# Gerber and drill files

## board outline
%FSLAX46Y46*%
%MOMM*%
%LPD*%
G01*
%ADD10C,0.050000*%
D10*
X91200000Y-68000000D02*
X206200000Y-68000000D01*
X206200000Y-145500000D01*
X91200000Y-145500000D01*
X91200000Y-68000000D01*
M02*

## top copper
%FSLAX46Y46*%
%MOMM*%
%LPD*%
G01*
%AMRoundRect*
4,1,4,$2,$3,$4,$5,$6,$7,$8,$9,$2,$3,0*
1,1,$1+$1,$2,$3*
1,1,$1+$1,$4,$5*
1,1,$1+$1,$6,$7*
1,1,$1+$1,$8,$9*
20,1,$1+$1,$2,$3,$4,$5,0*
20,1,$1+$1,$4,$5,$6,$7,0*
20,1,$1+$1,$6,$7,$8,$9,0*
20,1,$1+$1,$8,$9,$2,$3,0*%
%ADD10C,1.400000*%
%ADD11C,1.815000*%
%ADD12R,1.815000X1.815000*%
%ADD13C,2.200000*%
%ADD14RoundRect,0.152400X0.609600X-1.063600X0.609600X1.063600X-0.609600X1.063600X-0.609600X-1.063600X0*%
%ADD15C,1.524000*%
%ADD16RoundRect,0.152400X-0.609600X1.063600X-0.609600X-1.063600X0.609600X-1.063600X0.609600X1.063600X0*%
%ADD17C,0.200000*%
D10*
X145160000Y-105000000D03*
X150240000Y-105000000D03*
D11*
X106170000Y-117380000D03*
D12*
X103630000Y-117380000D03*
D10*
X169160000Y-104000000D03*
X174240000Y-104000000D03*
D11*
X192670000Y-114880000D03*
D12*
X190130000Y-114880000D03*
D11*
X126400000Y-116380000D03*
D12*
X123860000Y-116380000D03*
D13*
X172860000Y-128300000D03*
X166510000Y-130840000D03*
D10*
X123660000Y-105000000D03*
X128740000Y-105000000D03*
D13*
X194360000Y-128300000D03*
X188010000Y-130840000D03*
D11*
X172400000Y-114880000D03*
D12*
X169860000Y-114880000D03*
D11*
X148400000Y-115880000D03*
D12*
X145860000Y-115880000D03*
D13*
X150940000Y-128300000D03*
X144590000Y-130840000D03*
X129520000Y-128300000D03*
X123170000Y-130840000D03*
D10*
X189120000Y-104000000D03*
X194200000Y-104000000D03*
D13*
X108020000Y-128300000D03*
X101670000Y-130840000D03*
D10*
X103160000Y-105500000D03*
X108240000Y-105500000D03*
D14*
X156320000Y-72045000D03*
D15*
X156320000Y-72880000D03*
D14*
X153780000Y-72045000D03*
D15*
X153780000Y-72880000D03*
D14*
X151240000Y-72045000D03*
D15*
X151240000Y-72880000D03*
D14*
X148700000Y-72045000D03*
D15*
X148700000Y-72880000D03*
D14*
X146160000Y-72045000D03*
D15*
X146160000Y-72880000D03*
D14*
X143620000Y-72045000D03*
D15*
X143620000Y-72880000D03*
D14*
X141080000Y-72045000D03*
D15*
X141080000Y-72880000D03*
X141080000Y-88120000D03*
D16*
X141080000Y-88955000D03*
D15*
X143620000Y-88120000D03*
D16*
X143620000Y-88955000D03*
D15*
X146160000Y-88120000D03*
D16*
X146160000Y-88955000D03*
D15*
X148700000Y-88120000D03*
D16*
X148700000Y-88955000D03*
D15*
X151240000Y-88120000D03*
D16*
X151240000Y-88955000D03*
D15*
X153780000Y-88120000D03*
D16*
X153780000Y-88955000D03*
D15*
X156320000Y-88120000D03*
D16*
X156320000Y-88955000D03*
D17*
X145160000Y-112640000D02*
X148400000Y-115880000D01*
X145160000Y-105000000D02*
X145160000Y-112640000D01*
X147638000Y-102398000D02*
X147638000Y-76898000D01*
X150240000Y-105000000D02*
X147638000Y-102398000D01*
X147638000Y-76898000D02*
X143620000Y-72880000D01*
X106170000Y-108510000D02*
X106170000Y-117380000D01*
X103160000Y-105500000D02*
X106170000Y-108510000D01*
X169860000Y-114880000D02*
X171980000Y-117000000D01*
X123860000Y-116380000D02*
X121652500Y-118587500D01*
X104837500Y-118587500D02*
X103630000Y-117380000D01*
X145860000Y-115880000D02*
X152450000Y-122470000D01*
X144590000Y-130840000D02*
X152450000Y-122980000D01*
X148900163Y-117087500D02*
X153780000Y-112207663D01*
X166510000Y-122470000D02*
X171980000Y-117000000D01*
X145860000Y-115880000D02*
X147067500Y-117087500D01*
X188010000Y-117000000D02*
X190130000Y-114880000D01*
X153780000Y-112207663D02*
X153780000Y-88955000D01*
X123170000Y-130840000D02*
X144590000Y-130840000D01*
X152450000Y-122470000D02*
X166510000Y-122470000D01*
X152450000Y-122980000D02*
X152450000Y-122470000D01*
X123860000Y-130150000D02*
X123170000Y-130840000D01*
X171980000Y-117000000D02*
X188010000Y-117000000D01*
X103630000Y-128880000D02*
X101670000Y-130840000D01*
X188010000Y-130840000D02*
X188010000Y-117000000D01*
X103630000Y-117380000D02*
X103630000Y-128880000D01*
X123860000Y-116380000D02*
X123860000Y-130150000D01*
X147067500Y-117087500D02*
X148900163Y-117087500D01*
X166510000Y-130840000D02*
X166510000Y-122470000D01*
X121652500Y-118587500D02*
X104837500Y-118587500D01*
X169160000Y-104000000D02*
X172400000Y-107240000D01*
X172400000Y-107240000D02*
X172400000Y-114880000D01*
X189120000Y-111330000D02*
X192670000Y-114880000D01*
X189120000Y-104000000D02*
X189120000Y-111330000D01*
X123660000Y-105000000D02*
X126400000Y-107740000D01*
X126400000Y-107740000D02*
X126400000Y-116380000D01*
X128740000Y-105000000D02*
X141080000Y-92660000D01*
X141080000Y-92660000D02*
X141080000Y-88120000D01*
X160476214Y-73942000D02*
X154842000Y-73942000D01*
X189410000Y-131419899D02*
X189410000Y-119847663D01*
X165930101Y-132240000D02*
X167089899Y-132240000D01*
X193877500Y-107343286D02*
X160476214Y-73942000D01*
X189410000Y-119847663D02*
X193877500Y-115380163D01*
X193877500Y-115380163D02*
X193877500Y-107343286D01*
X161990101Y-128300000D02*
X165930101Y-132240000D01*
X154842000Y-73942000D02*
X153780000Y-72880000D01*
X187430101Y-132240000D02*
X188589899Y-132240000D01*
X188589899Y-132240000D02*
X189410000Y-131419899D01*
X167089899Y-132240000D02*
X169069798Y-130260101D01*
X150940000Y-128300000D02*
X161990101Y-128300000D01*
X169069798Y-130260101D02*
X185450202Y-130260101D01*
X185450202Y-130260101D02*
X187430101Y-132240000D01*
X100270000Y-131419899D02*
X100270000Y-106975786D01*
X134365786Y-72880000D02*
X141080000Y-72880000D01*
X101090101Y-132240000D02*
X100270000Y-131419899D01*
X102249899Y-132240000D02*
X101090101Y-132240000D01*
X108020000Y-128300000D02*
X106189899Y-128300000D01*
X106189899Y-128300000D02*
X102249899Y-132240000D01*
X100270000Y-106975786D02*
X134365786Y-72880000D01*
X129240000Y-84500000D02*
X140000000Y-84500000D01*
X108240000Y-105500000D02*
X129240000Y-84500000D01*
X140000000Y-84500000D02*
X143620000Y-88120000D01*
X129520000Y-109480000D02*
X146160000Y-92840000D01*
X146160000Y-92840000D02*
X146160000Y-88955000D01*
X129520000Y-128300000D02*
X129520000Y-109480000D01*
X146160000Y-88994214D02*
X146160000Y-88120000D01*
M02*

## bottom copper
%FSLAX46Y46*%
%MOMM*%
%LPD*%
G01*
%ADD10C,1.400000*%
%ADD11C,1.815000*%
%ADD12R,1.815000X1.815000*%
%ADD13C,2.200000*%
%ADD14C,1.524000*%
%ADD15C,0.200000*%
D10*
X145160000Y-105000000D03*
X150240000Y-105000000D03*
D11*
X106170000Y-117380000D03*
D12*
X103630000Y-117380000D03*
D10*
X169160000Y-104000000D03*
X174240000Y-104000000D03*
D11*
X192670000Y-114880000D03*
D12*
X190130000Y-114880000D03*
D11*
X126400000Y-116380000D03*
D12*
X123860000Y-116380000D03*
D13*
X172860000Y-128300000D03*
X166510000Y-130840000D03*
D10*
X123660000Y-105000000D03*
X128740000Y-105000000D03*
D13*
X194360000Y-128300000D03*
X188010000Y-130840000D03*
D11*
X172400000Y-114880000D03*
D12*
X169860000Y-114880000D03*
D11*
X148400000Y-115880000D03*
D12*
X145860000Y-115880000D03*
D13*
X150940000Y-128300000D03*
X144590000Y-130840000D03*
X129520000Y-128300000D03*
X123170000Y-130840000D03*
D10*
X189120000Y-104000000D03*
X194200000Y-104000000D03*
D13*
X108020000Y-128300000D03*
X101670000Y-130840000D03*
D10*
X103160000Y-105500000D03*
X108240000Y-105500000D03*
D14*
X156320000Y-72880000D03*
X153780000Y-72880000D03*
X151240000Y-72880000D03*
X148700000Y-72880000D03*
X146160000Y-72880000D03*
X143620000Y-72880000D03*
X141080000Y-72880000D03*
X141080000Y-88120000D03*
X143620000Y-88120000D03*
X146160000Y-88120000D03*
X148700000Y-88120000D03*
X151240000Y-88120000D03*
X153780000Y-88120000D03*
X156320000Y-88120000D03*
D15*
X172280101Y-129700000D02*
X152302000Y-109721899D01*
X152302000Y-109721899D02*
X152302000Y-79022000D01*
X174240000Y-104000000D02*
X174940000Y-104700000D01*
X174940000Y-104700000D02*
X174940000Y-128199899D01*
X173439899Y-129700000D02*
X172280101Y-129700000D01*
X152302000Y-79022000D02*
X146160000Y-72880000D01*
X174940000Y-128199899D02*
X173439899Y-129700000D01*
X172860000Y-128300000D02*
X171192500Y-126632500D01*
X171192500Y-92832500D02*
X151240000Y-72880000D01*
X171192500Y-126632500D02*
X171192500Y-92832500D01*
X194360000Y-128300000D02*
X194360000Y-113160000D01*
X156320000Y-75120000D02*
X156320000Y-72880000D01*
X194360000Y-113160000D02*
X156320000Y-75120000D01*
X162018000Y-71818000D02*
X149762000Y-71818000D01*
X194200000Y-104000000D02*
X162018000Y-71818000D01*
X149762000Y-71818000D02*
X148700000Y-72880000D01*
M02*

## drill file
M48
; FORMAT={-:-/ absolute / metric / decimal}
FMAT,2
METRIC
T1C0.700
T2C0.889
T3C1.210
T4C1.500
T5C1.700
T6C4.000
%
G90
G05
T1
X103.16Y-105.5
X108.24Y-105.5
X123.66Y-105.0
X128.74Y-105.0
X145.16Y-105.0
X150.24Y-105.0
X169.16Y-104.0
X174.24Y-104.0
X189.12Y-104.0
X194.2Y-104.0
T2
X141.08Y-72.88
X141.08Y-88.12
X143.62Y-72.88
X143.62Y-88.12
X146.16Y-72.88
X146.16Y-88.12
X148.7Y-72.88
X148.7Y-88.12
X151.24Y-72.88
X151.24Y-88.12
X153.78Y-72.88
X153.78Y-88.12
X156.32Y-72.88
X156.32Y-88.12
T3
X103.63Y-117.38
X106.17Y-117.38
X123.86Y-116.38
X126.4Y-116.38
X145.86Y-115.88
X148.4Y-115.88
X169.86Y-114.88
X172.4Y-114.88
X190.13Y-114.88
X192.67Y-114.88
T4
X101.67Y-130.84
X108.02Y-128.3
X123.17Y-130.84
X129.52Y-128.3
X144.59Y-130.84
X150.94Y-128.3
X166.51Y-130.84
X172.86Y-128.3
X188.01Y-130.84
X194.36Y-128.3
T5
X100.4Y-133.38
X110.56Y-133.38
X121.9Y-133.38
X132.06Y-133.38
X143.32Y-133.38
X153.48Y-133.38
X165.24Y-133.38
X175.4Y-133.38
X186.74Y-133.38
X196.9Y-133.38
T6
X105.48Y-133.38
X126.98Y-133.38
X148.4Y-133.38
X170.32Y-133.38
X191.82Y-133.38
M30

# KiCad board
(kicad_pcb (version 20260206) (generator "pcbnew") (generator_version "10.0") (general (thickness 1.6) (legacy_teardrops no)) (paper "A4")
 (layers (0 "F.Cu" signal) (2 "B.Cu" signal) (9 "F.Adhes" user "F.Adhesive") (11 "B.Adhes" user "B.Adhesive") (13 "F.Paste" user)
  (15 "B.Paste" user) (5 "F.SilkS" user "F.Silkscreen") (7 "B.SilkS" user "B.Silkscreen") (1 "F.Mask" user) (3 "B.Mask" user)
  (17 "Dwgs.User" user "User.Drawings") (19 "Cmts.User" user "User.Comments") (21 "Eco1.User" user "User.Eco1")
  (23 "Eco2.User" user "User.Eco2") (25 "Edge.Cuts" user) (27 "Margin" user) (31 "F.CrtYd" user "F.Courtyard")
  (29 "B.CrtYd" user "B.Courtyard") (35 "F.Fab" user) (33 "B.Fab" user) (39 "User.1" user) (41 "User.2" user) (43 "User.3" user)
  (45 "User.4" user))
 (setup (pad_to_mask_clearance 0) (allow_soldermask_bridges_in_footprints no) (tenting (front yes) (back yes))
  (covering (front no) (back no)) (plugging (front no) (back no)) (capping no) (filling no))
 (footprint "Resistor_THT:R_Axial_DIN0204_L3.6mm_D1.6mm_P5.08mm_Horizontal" (layer "F.Cu") (at 145.16 105)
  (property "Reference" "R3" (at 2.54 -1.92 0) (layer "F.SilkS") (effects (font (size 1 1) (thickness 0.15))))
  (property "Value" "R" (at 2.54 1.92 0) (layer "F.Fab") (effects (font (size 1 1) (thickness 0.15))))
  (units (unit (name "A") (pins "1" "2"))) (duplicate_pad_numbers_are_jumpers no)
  (pad "1" thru_hole circle (at 0 0) (size 1.4 1.4) (drill 0.7) (layers "*.Cu" "*.Mask") (remove_unused_layers no) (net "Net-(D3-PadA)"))
  (pad "2" thru_hole circle (at 5.08 0) (size 1.4 1.4) (drill 0.7) (layers "*.Cu" "*.Mask") (remove_unused_layers no)
   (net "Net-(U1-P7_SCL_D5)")))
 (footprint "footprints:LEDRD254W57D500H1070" (layer "F.Cu") (at 104.9 117.38)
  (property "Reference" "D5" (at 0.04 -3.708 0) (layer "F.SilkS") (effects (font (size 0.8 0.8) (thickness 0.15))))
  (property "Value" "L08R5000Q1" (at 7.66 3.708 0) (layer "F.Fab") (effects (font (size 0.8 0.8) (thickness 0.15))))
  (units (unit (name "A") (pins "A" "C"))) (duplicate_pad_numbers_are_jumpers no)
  (pad "A" thru_hole circle (at 1.27 0) (size 1.815 1.815) (drill 1.21) (layers "*.Cu" "*.Mask") (remove_unused_layers no)
   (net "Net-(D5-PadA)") (solder_mask_margin 0.102))
  (pad "C" thru_hole rect (at -1.27 0) (size 1.815 1.815) (drill 1.21) (layers "*.Cu" "*.Mask") (remove_unused_layers no) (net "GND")
   (solder_mask_margin 0.102)))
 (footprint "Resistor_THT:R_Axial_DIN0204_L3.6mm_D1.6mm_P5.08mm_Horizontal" (layer "F.Cu") (at 169.16 104)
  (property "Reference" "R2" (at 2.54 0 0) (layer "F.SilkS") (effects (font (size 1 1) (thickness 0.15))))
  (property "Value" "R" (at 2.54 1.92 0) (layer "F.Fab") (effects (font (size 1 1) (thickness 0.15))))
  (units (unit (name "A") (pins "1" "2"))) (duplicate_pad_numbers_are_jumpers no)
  (pad "1" thru_hole circle (at 0 0) (size 1.4 1.4) (drill 0.7) (layers "*.Cu" "*.Mask") (remove_unused_layers no) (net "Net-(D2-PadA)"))
  (pad "2" thru_hole circle (at 5.08 0) (size 1.4 1.4) (drill 0.7) (layers "*.Cu" "*.Mask") (remove_unused_layers no)
   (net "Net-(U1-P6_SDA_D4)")))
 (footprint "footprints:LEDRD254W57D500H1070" (layer "F.Cu") (at 191.4 114.88)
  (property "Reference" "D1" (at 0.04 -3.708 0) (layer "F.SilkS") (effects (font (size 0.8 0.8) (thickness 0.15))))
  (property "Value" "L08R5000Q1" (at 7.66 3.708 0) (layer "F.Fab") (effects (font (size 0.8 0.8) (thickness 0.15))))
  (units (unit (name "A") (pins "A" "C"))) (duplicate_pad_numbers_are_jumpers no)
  (pad "A" thru_hole circle (at 1.27 0) (size 1.815 1.815) (drill 1.21) (layers "*.Cu" "*.Mask") (remove_unused_layers no)
   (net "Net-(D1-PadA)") (solder_mask_margin 0.102))
  (pad "C" thru_hole rect (at -1.27 0) (size 1.815 1.815) (drill 1.21) (layers "*.Cu" "*.Mask") (remove_unused_layers no) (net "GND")
   (solder_mask_margin 0.102)))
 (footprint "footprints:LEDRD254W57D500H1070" (layer "F.Cu") (at 125.13 116.38)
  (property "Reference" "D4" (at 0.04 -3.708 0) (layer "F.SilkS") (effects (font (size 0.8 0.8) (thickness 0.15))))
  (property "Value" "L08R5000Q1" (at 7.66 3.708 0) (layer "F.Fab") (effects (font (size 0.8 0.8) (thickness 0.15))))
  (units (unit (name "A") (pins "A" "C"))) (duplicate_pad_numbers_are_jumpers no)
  (pad "A" thru_hole circle (at 1.27 0) (size 1.815 1.815) (drill 1.21) (layers "*.Cu" "*.Mask") (remove_unused_layers no)
   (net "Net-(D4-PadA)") (solder_mask_margin 0.102))
  (pad "C" thru_hole rect (at -1.27 0) (size 1.815 1.815) (drill 1.21) (layers "*.Cu" "*.Mask") (remove_unused_layers no) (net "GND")
   (solder_mask_margin 0.102)))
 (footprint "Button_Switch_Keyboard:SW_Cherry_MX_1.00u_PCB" (layer "F.Cu") (at 172.86 128.3)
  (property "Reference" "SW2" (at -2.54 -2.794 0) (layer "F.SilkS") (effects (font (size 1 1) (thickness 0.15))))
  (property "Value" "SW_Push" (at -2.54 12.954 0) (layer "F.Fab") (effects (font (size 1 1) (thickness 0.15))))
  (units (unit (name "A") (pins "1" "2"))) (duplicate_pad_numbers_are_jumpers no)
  (pad "" np_thru_hole circle (at -7.62 5.08) (size 1.7 1.7) (drill 1.7) (layers "*.Cu" "*.Mask"))
  (pad "" np_thru_hole circle (at -2.54 5.08) (size 4 4) (drill 4) (layers "*.Cu" "*.Mask"))
  (pad "" np_thru_hole circle (at 2.54 5.08) (size 1.7 1.7) (drill 1.7) (layers "*.Cu" "*.Mask"))
  (pad "1" thru_hole circle (at 0 0) (size 2.2 2.2) (drill 1.5) (layers "*.Cu" "*.Mask") (remove_unused_layers no)
   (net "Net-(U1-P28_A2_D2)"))
  (pad "2" thru_hole circle (at -6.35 2.54) (size 2.2 2.2) (drill 1.5) (layers "*.Cu" "*.Mask") (remove_unused_layers no) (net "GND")))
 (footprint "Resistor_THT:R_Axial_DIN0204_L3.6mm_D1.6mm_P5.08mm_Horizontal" (layer "F.Cu") (at 123.66 105)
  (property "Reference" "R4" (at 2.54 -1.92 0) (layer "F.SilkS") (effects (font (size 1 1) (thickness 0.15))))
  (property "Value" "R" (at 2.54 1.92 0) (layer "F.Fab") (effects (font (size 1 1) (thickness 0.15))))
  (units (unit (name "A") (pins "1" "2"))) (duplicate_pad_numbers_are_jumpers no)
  (pad "1" thru_hole circle (at 0 0) (size 1.4 1.4) (drill 0.7) (layers "*.Cu" "*.Mask") (remove_unused_layers no) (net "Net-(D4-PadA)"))
  (pad "2" thru_hole circle (at 5.08 0) (size 1.4 1.4) (drill 0.7) (layers "*.Cu" "*.Mask") (remove_unused_layers no)
   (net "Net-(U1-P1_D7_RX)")))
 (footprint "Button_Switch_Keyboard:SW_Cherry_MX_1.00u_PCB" (layer "F.Cu") (at 194.36 128.3)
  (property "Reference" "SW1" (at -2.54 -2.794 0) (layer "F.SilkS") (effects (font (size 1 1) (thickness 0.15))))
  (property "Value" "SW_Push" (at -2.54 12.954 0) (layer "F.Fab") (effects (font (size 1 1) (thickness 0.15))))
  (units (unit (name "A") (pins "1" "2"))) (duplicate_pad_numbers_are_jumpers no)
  (pad "" np_thru_hole circle (at -7.62 5.08) (size 1.7 1.7) (drill 1.7) (layers "*.Cu" "*.Mask"))
  (pad "" np_thru_hole circle (at -2.54 5.08) (size 4 4) (drill 4) (layers "*.Cu" "*.Mask"))
  (pad "" np_thru_hole circle (at 2.54 5.08) (size 1.7 1.7) (drill 1.7) (layers "*.Cu" "*.Mask"))
  (pad "1" thru_hole circle (at 0 0) (size 2.2 2.2) (drill 1.5) (layers "*.Cu" "*.Mask") (remove_unused_layers no)
   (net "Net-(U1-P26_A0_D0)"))
  (pad "2" thru_hole circle (at -6.35 2.54) (size 2.2 2.2) (drill 1.5) (layers "*.Cu" "*.Mask") (remove_unused_layers no) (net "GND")))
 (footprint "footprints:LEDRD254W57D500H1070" (layer "F.Cu") (at 171.13 114.88)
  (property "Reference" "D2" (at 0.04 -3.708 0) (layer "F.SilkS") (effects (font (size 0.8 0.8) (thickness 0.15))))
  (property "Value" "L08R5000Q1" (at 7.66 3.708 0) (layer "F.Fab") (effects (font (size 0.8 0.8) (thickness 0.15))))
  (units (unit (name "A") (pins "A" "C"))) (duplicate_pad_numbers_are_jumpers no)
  (pad "A" thru_hole circle (at 1.27 0) (size 1.815 1.815) (drill 1.21) (layers "*.Cu" "*.Mask") (remove_unused_layers no)
   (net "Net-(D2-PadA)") (solder_mask_margin 0.102))
  (pad "C" thru_hole rect (at -1.27 0) (size 1.815 1.815) (drill 1.21) (layers "*.Cu" "*.Mask") (remove_unused_layers no) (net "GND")
   (solder_mask_margin 0.102)))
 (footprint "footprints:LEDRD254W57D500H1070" (layer "F.Cu") (at 147.13 115.88)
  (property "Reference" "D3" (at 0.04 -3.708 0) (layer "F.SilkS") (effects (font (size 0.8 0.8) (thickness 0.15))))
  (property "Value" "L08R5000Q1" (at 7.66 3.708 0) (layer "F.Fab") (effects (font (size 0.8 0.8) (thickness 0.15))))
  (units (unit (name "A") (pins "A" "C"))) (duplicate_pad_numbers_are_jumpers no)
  (pad "A" thru_hole circle (at 1.27 0) (size 1.815 1.815) (drill 1.21) (layers "*.Cu" "*.Mask") (remove_unused_layers no)
   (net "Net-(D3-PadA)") (solder_mask_margin 0.102))
  (pad "C" thru_hole rect (at -1.27 0) (size 1.815 1.815) (drill 1.21) (layers "*.Cu" "*.Mask") (remove_unused_layers no) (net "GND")
   (solder_mask_margin 0.102)))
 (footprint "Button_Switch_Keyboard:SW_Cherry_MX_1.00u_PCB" (layer "F.Cu") (at 150.94 128.3)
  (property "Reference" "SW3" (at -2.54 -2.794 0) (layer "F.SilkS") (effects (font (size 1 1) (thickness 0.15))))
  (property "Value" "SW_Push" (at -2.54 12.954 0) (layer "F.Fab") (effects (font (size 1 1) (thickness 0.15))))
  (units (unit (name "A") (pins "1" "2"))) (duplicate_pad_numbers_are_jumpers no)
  (pad "" np_thru_hole circle (at -7.62 5.08) (size 1.7 1.7) (drill 1.7) (layers "*.Cu" "*.Mask"))
  (pad "" np_thru_hole circle (at -2.54 5.08) (size 4 4) (drill 4) (layers "*.Cu" "*.Mask"))
  (pad "" np_thru_hole circle (at 2.54 5.08) (size 1.7 1.7) (drill 1.7) (layers "*.Cu" "*.Mask"))
  (pad "1" thru_hole circle (at 0 0) (size 2.2 2.2) (drill 1.5) (layers "*.Cu" "*.Mask") (remove_unused_layers no)
   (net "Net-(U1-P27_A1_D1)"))
  (pad "2" thru_hole circle (at -6.35 2.54) (size 2.2 2.2) (drill 1.5) (layers "*.Cu" "*.Mask") (remove_unused_layers no) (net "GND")))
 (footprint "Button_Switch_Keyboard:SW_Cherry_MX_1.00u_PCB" (layer "F.Cu") (at 129.52 128.3)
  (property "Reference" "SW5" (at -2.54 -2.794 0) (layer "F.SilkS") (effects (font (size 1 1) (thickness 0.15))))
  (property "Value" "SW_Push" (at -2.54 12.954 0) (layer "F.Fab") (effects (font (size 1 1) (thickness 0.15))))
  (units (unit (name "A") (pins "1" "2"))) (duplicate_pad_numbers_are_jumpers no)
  (pad "" np_thru_hole circle (at -7.62 5.08) (size 1.7 1.7) (drill 1.7) (layers "*.Cu" "*.Mask"))
  (pad "" np_thru_hole circle (at -2.54 5.08) (size 4 4) (drill 4) (layers "*.Cu" "*.Mask"))
  (pad "" np_thru_hole circle (at 2.54 5.08) (size 1.7 1.7) (drill 1.7) (layers "*.Cu" "*.Mask"))
  (pad "1" thru_hole circle (at 0 0) (size 2.2 2.2) (drill 1.5) (layers "*.Cu" "*.Mask") (remove_unused_layers no)
   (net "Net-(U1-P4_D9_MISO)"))
  (pad "2" thru_hole circle (at -6.35 2.54) (size 2.2 2.2) (drill 1.5) (layers "*.Cu" "*.Mask") (remove_unused_layers no) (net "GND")))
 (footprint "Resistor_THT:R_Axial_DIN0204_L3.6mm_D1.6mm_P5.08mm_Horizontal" (layer "F.Cu") (at 189.12 104)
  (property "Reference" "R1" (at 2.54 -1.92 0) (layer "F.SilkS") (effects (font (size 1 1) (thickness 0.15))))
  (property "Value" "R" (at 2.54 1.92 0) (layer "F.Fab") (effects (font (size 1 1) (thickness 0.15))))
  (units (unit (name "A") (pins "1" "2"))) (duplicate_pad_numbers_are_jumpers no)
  (pad "1" thru_hole circle (at 0 0) (size 1.4 1.4) (drill 0.7) (layers "*.Cu" "*.Mask") (remove_unused_layers no) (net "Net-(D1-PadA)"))
  (pad "2" thru_hole circle (at 5.08 0) (size 1.4 1.4) (drill 0.7) (layers "*.Cu" "*.Mask") (remove_unused_layers no)
   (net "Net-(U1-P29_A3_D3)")))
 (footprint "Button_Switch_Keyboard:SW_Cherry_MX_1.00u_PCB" (layer "F.Cu") (at 108.02 128.3)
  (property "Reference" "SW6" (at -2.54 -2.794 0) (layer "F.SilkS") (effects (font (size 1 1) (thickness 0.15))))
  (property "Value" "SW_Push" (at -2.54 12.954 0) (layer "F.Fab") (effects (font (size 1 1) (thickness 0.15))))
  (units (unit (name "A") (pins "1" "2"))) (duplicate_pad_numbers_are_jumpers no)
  (pad "" np_thru_hole circle (at -7.62 5.08) (size 1.7 1.7) (drill 1.7) (layers "*.Cu" "*.Mask"))
  (pad "" np_thru_hole circle (at -2.54 5.08) (size 4 4) (drill 4) (layers "*.Cu" "*.Mask"))
  (pad "" np_thru_hole circle (at 2.54 5.08) (size 1.7 1.7) (drill 1.7) (layers "*.Cu" "*.Mask"))
  (pad "1" thru_hole circle (at 0 0) (size 2.2 2.2) (drill 1.5) (layers "*.Cu" "*.Mask") (remove_unused_layers no) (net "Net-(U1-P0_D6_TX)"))
  (pad "2" thru_hole circle (at -6.35 2.54) (size 2.2 2.2) (drill 1.5) (layers "*.Cu" "*.Mask") (remove_unused_layers no) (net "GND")))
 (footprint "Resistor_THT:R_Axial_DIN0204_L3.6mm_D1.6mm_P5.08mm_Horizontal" (layer "F.Cu") (at 103.16 105.5)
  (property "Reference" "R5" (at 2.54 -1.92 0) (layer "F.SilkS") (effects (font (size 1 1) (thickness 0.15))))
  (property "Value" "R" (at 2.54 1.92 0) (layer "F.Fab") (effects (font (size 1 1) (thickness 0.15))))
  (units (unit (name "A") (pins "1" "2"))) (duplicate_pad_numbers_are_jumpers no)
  (pad "1" thru_hole circle (at 0 0) (size 1.4 1.4) (drill 0.7) (layers "*.Cu" "*.Mask") (remove_unused_layers no) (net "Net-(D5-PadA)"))
  (pad "2" thru_hole circle (at 5.08 0) (size 1.4 1.4) (drill 0.7) (layers "*.Cu" "*.Mask") (remove_unused_layers no)
   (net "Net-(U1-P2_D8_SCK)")))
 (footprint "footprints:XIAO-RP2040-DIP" (layer "F.Cu") (at 148.7 80.5)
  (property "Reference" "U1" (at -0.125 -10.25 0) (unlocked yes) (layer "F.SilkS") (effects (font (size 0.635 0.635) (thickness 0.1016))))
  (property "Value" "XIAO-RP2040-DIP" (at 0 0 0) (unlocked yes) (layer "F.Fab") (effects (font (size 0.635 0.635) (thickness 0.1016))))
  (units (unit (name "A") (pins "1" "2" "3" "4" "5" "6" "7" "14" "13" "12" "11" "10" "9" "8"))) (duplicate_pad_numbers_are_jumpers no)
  (pad "1" smd roundrect (at 7.62 -8.455 90) (size 2.432 1.524) (layers "F.Cu" "F.Mask") (roundrect_rratio 0.1) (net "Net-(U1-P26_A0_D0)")
   (thermal_bridge_angle 45))
  (pad "1" thru_hole circle (at 7.62 -7.62 90) (size 1.524 1.524) (drill 0.889) (layers "*.Cu" "*.Mask") (remove_unused_layers no)
   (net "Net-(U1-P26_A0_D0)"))
  (pad "2" smd roundrect (at 5.08 -8.455 90) (size 2.432 1.524) (layers "F.Cu" "F.Mask") (roundrect_rratio 0.1) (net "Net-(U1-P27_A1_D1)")
   (thermal_bridge_angle 45))
  (pad "2" thru_hole circle (at 5.08 -7.62 90) (size 1.524 1.524) (drill 0.889) (layers "*.Cu" "*.Mask") (remove_unused_layers no)
   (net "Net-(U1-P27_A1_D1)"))
  (pad "3" smd roundrect (at 2.54 -8.455 90) (size 2.432 1.524) (layers "F.Cu" "F.Mask") (roundrect_rratio 0.1) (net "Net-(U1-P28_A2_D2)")
   (thermal_bridge_angle 45))
  (pad "3" thru_hole circle (at 2.54 -7.62 90) (size 1.524 1.524) (drill 0.889) (layers "*.Cu" "*.Mask") (remove_unused_layers no)
   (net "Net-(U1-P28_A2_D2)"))
  (pad "4" smd roundrect (at 0 -8.455 90) (size 2.432 1.524) (layers "F.Cu" "F.Mask") (roundrect_rratio 0.1) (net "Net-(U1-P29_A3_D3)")
   (thermal_bridge_angle 45))
  (pad "4" thru_hole circle (at 0 -7.62 90) (size 1.524 1.524) (drill 0.889) (layers "*.Cu" "*.Mask") (remove_unused_layers no)
   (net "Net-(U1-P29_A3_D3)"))
  (pad "5" smd roundrect (at -2.54 -8.455 90) (size 2.432 1.524) (layers "F.Cu" "F.Mask") (roundrect_rratio 0.1) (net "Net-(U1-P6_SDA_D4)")
   (thermal_bridge_angle 45))
  (pad "5" thru_hole circle (at -2.54 -7.62 90) (size 1.524 1.524) (drill 0.889) (layers "*.Cu" "*.Mask") (remove_unused_layers no)
   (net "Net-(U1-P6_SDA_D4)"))
  (pad "6" smd roundrect (at -5.08 -8.455 90) (size 2.432 1.524) (layers "F.Cu" "F.Mask") (roundrect_rratio 0.1) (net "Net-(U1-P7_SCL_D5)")
   (thermal_bridge_angle 45))
  (pad "6" thru_hole circle (at -5.08 -7.62 90) (size 1.524 1.524) (drill 0.889) (layers "*.Cu" "*.Mask") (remove_unused_layers no)
   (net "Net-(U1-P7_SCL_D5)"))
  (pad "7" smd roundrect (at -7.62 -8.455 90) (size 2.432 1.524) (layers "F.Cu" "F.Mask") (roundrect_rratio 0.1) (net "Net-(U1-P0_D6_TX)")
   (thermal_bridge_angle 45))
  (pad "7" thru_hole circle (at -7.62 -7.62 90) (size 1.524 1.524) (drill 0.889) (layers "*.Cu" "*.Mask") (remove_unused_layers no)
   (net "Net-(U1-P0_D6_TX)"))
  (pad "8" thru_hole circle (at -7.62 7.62 270) (size 1.524 1.524) (drill 0.889) (layers "*.Cu" "*.Mask") (remove_unused_layers no)
   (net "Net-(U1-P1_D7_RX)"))
  (pad "8" smd roundrect (at -7.62 8.455 270) (size 2.432 1.524) (layers "F.Cu" "F.Mask") (roundrect_rratio 0.1) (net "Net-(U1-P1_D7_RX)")
   (thermal_bridge_angle 45))
  (pad "9" thru_hole circle (at -5.08 7.62 270) (size 1.524 1.524) (drill 0.889) (layers "*.Cu" "*.Mask") (remove_unused_layers no)
   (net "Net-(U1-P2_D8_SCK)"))
  (pad "9" smd roundrect (at -5.08 8.455 270) (size 2.432 1.524) (layers "F.Cu" "F.Mask") (roundrect_rratio 0.1) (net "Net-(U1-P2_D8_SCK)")
   (thermal_bridge_angle 45))
  (pad "10" thru_hole circle (at -2.54 7.62 270) (size 1.524 1.524) (drill 0.889) (layers "*.Cu" "*.Mask") (remove_unused_layers no)
   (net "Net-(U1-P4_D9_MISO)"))
  (pad "10" smd roundrect (at -2.54 8.455 270) (size 2.432 1.524) (layers "F.Cu" "F.Mask") (roundrect_rratio 0.1)
   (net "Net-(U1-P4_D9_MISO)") (thermal_bridge_angle 45))
  (pad "11" thru_hole circle (at 0 7.62 270) (size 1.524 1.524) (drill 0.889) (layers "*.Cu" "*.Mask") (remove_unused_layers no)
   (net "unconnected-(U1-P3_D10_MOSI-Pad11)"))
  (pad "11" smd roundrect (at 0 8.455 270) (size 2.432 1.524) (layers "F.Cu" "F.Mask") (roundrect_rratio 0.1)
   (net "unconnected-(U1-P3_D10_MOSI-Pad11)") (thermal_bridge_angle 45))
  (pad "12" thru_hole circle (at 2.54 7.62 270) (size 1.524 1.524) (drill 0.889) (layers "*.Cu" "*.Mask") (remove_unused_layers no)
   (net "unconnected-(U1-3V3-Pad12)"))
  (pad "12" smd roundrect (at 2.54 8.455 270) (size 2.432 1.524) (layers "F.Cu" "F.Mask") (roundrect_rratio 0.1)
   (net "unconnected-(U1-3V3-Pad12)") (thermal_bridge_angle 45))
  (pad "13" thru_hole circle (at 5.08 7.62 270) (size 1.524 1.524) (drill 0.889) (layers "*.Cu" "*.Mask") (remove_unused_layers no)
   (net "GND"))
  (pad "13" smd roundrect (at 5.08 8.455 270) (size 2.432 1.524) (layers "F.Cu" "F.Mask") (roundrect_rratio 0.1) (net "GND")
   (thermal_bridge_angle 45))
  (pad "14" thru_hole circle (at 7.62 7.62 270) (size 1.524 1.524) (drill 0.889) (layers "*.Cu" "*.Mask") (remove_unused_layers no)
   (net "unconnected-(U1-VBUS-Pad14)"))
  (pad "14" smd roundrect (at 7.62 8.455 270) (size 2.432 1.524) (layers "F.Cu" "F.Mask") (roundrect_rratio 0.1)
   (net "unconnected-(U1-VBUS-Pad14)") (thermal_bridge_angle 45)))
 (gr_rect (start 91.2 68) (end 206.2 145.5) (stroke (width 0.05) (type default)) (fill no) (layer "Edge.Cuts"))
 (segment (start 145.16 112.64) (end 148.4 115.88) (width 0.2) (layer "F.Cu") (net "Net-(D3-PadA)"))
 (segment (start 145.16 105) (end 145.16 112.64) (width 0.2) (layer "F.Cu") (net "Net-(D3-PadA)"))
 (segment (start 147.638 102.398) (end 147.638 76.898) (width 0.2) (layer "F.Cu") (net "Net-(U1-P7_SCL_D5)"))
 (segment (start 150.24 105) (end 147.638 102.398) (width 0.2) (layer "F.Cu") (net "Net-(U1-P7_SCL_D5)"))
 (segment (start 147.638 76.898) (end 143.62 72.88) (width 0.2) (layer "F.Cu") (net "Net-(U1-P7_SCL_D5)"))
 (segment (start 106.17 108.51) (end 106.17 117.38) (width 0.2) (layer "F.Cu") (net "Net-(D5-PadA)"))
 (segment (start 103.16 105.5) (end 106.17 108.51) (width 0.2) (layer "F.Cu") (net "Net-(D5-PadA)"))
 (segment (start 169.86 114.88) (end 171.98 117) (width 0.2) (layer "F.Cu") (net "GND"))
 (segment (start 123.86 116.38) (end 121.6525 118.5875) (width 0.2) (layer "F.Cu") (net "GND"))
 (segment (start 104.8375 118.5875) (end 103.63 117.38) (width 0.2) (layer "F.Cu") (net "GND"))
 (segment (start 145.86 115.88) (end 152.45 122.47) (width 0.2) (layer "F.Cu") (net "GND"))
 (segment (start 144.59 130.84) (end 152.45 122.98) (width 0.2) (layer "F.Cu") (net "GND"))
 (segment (start 148.900163 117.0875) (end 153.78 112.207663) (width 0.2) (layer "F.Cu") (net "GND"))
 (segment (start 166.51 122.47) (end 171.98 117) (width 0.2) (layer "F.Cu") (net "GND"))
 (segment (start 145.86 115.88) (end 147.0675 117.0875) (width 0.2) (layer "F.Cu") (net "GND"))
 (segment (start 188.01 117) (end 190.13 114.88) (width 0.2) (layer "F.Cu") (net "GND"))
 (segment (start 153.78 112.207663) (end 153.78 88.955) (width 0.2) (layer "F.Cu") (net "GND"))
 (segment (start 123.17 130.84) (end 144.59 130.84) (width 0.2) (layer "F.Cu") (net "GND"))
 (segment (start 152.45 122.47) (end 166.51 122.47) (width 0.2) (layer "F.Cu") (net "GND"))
 (segment (start 152.45 122.98) (end 152.45 122.47) (width 0.2) (layer "F.Cu") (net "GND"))
 (segment (start 123.86 130.15) (end 123.17 130.84) (width 0.2) (layer "F.Cu") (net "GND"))
 (segment (start 171.98 117) (end 188.01 117) (width 0.2) (layer "F.Cu") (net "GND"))
 (segment (start 103.63 128.88) (end 101.67 130.84) (width 0.2) (layer "F.Cu") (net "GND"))
 (segment (start 188.01 130.84) (end 188.01 117) (width 0.2) (layer "F.Cu") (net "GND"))
 (segment (start 103.63 117.38) (end 103.63 128.88) (width 0.2) (layer "F.Cu") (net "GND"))
 (segment (start 123.86 116.38) (end 123.86 130.15) (width 0.2) (layer "F.Cu") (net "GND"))
 (segment (start 147.0675 117.0875) (end 148.900163 117.0875) (width 0.2) (layer "F.Cu") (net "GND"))
 (segment (start 166.51 130.84) (end 166.51 122.47) (width 0.2) (layer "F.Cu") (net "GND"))
 (segment (start 121.6525 118.5875) (end 104.8375 118.5875) (width 0.2) (layer "F.Cu") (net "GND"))
 (segment (start 169.16 104) (end 172.4 107.24) (width 0.2) (layer "F.Cu") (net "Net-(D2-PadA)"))
 (segment (start 172.4 107.24) (end 172.4 114.88) (width 0.2) (layer "F.Cu") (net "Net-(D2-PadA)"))
 (segment (start 172.280101 129.7) (end 152.302 109.721899) (width 0.2) (layer "B.Cu") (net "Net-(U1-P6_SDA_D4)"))
 (segment (start 152.302 109.721899) (end 152.302 79.022) (width 0.2) (layer "B.Cu") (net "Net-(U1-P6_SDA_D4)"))
 (segment (start 174.24 104) (end 174.94 104.7) (width 0.2) (layer "B.Cu") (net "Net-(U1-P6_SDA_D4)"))
 (segment (start 174.94 104.7) (end 174.94 128.199899) (width 0.2) (layer "B.Cu") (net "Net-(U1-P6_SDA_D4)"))
 (segment (start 173.439899 129.7) (end 172.280101 129.7) (width 0.2) (layer "B.Cu") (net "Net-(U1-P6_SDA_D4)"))
 (segment (start 152.302 79.022) (end 146.16 72.88) (width 0.2) (layer "B.Cu") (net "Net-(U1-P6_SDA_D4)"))
 (segment (start 174.94 128.199899) (end 173.439899 129.7) (width 0.2) (layer "B.Cu") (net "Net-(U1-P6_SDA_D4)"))
 (segment (start 189.12 111.33) (end 192.67 114.88) (width 0.2) (layer "F.Cu") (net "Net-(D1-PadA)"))
 (segment (start 189.12 104) (end 189.12 111.33) (width 0.2) (layer "F.Cu") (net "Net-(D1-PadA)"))
 (segment (start 123.66 105) (end 126.4 107.74) (width 0.2) (layer "F.Cu") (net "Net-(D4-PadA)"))
 (segment (start 126.4 107.74) (end 126.4 116.38) (width 0.2) (layer "F.Cu") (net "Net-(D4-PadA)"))
 (segment (start 172.86 128.3) (end 171.1925 126.6325) (width 0.2) (layer "B.Cu") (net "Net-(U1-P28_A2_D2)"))
 (segment (start 171.1925 92.8325) (end 151.24 72.88) (width 0.2) (layer "B.Cu") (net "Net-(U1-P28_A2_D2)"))
 (segment (start 171.1925 126.6325) (end 171.1925 92.8325) (width 0.2) (layer "B.Cu") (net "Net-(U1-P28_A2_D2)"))
 (segment (start 128.74 105) (end 141.08 92.66) (width 0.2) (layer "F.Cu") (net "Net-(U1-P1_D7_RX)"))
 (segment (start 141.08 92.66) (end 141.08 88.12) (width 0.2) (layer "F.Cu") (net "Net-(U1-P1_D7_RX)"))
 (segment (start 194.36 128.3) (end 194.36 113.16) (width 0.2) (layer "B.Cu") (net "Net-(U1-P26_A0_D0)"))
 (segment (start 156.32 75.12) (end 156.32 72.88) (width 0.2) (layer "B.Cu") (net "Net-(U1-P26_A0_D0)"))
 (segment (start 194.36 113.16) (end 156.32 75.12) (width 0.2) (layer "B.Cu") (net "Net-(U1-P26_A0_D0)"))
 (segment (start 160.476214 73.942) (end 154.842 73.942) (width 0.2) (layer "F.Cu") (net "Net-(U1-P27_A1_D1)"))
 (segment (start 189.41 131.419899) (end 189.41 119.847663) (width 0.2) (layer "F.Cu") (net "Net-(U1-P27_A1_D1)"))
 (segment (start 165.930101 132.24) (end 167.089899 132.24) (width 0.2) (layer "F.Cu") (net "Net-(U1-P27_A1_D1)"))
 (segment (start 193.8775 107.343286) (end 160.476214 73.942) (width 0.2) (layer "F.Cu") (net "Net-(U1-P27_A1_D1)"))
 (segment (start 189.41 119.847663) (end 193.8775 115.380163) (width 0.2) (layer "F.Cu") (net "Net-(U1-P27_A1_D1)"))
 (segment (start 193.8775 115.380163) (end 193.8775 107.343286) (width 0.2) (layer "F.Cu") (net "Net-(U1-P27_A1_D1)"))
 (segment (start 161.990101 128.3) (end 165.930101 132.24) (width 0.2) (layer "F.Cu") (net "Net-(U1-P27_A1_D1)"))
 (segment (start 154.842 73.942) (end 153.78 72.88) (width 0.2) (layer "F.Cu") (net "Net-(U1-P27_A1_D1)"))
 (segment (start 187.430101 132.24) (end 188.589899 132.24) (width 0.2) (layer "F.Cu") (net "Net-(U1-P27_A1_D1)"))
 (segment (start 188.589899 132.24) (end 189.41 131.419899) (width 0.2) (layer "F.Cu") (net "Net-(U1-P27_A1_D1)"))
 (segment (start 167.089899 132.24) (end 169.069798 130.260101) (width 0.2) (layer "F.Cu") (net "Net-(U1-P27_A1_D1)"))
 (segment (start 150.94 128.3) (end 161.990101 128.3) (width 0.2) (layer "F.Cu") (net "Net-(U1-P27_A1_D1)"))
 (segment (start 169.069798 130.260101) (end 185.450202 130.260101) (width 0.2) (layer "F.Cu") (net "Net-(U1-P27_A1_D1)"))
 (segment (start 185.450202 130.260101) (end 187.430101 132.24) (width 0.2) (layer "F.Cu") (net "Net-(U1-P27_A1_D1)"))
 (segment (start 162.018 71.818) (end 149.762 71.818) (width 0.2) (layer "B.Cu") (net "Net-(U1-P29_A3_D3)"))
 (segment (start 194.2 104) (end 162.018 71.818) (width 0.2) (layer "B.Cu") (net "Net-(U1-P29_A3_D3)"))
 (segment (start 149.762 71.818) (end 148.7 72.88) (width 0.2) (layer "B.Cu") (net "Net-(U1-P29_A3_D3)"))
 (segment (start 100.27 131.419899) (end 100.27 106.975786) (width 0.2) (layer "F.Cu") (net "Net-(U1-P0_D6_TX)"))
 (segment (start 134.365786 72.88) (end 141.08 72.88) (width 0.2) (layer "F.Cu") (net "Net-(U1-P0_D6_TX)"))
 (segment (start 101.090101 132.24) (end 100.27 131.419899) (width 0.2) (layer "F.Cu") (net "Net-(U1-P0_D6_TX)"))
 (segment (start 102.249899 132.24) (end 101.090101 132.24) (width 0.2) (layer "F.Cu") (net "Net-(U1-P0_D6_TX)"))
 (segment (start 108.02 128.3) (end 106.189899 128.3) (width 0.2) (layer "F.Cu") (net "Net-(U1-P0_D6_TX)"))
 (segment (start 106.189899 128.3) (end 102.249899 132.24) (width 0.2) (layer "F.Cu") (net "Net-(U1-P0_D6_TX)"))
 (segment (start 100.27 106.975786) (end 134.365786 72.88) (width 0.2) (layer "F.Cu") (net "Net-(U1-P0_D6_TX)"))
 (segment (start 129.24 84.5) (end 140 84.5) (width 0.2) (layer "F.Cu") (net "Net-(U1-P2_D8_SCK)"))
 (segment (start 108.24 105.5) (end 129.24 84.5) (width 0.2) (layer "F.Cu") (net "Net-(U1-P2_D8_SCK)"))
 (segment (start 140 84.5) (end 143.62 88.12) (width 0.2) (layer "F.Cu") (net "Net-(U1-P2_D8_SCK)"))
 (segment (start 129.52 109.48) (end 146.16 92.84) (width 0.2) (layer "F.Cu") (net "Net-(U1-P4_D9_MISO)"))
 (segment (start 146.16 92.84) (end 146.16 88.955) (width 0.2) (layer "F.Cu") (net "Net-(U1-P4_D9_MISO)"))
 (segment (start 129.52 128.3) (end 129.52 109.48) (width 0.2) (layer "F.Cu") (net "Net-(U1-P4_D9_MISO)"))
 (segment (start 146.16 88.994214) (end 146.16 88.12) (width 0.2) (layer "F.Cu") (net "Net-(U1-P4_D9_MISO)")))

